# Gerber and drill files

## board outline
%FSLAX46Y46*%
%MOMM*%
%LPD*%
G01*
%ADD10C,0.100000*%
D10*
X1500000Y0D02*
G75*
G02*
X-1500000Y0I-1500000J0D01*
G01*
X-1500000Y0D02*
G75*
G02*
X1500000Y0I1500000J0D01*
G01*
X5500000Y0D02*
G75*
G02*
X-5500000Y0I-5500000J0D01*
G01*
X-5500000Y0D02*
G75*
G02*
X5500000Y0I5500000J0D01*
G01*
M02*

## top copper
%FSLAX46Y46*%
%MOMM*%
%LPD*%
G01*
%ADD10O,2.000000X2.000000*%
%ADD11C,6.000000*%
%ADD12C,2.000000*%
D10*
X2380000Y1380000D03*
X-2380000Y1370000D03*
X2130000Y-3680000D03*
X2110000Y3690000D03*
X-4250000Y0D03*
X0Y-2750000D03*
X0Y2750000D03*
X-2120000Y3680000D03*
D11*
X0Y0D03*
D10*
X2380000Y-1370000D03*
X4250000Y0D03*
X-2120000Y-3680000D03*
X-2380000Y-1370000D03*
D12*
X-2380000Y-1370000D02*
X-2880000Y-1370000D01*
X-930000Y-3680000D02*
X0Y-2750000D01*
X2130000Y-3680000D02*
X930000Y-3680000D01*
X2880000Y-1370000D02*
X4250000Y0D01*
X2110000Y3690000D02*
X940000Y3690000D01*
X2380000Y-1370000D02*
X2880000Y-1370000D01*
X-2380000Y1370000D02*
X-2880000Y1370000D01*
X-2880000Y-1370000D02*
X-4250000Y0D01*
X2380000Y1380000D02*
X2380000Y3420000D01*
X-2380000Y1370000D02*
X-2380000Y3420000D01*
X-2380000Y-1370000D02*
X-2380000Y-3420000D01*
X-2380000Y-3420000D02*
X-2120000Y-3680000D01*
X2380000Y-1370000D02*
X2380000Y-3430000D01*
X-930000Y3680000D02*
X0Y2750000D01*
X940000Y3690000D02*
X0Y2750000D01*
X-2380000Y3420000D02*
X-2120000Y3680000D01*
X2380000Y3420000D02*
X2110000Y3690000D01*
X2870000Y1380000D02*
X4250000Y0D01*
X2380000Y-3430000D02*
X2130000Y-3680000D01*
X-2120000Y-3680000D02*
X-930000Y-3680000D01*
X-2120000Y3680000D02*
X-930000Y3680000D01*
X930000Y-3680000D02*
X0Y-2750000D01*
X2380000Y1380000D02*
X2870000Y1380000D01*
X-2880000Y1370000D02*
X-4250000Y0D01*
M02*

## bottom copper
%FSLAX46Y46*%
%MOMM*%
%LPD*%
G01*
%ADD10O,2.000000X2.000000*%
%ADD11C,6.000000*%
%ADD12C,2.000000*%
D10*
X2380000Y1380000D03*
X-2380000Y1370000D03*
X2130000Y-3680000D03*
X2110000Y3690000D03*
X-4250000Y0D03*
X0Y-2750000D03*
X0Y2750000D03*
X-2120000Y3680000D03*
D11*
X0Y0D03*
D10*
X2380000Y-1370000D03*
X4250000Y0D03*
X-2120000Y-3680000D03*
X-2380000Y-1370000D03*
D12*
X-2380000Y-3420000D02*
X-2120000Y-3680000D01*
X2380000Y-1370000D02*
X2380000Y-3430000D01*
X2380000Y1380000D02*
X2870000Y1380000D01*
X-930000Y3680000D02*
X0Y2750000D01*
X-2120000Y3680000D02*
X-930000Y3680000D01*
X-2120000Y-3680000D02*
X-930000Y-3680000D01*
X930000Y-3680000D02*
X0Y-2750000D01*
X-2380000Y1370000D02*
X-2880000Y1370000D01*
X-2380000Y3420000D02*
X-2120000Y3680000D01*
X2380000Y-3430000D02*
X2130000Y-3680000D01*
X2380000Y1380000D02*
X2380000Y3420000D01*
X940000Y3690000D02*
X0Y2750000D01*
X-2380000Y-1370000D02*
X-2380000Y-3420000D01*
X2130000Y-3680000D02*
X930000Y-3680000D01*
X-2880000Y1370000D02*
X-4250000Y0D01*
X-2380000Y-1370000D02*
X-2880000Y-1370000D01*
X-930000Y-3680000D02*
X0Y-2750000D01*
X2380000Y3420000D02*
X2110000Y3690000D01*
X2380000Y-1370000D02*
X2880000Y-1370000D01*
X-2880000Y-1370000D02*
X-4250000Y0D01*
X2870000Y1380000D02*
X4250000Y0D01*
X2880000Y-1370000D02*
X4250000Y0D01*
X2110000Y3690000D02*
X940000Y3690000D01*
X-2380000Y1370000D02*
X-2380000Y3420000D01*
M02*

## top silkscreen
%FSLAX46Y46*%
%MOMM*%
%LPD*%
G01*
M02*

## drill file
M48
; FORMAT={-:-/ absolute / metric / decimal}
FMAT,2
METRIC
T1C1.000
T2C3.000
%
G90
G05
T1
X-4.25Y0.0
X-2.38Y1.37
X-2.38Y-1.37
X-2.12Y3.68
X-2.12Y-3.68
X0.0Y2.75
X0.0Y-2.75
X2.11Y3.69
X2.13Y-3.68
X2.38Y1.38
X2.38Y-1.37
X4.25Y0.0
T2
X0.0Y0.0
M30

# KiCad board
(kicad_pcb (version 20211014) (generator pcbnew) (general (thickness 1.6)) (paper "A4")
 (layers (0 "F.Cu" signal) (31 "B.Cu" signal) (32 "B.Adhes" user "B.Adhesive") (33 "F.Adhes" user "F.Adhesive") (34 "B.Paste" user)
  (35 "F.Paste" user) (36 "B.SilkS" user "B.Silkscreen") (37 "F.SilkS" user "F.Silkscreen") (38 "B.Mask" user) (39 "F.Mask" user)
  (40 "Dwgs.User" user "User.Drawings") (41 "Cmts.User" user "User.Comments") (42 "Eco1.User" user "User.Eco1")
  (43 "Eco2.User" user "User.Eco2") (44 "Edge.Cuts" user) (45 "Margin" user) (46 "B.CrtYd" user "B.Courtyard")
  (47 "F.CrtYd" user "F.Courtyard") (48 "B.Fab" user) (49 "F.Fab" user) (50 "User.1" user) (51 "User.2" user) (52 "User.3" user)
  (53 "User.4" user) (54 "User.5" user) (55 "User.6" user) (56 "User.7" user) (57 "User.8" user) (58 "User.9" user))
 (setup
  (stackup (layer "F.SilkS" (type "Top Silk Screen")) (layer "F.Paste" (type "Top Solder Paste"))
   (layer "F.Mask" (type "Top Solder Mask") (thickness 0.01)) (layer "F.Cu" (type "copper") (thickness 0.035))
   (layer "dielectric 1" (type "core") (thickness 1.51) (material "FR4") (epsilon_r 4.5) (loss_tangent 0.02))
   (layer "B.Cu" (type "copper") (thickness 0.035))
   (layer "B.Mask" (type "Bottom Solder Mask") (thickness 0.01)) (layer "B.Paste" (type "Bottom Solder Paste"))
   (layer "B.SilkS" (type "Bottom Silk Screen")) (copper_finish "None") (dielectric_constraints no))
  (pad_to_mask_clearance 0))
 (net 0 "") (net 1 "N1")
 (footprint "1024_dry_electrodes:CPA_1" (layer "F.Cu") (at 2.38 -1.38)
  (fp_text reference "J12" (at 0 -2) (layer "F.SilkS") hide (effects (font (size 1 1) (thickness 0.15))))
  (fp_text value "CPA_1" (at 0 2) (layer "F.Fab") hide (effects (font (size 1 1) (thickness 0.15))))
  (pad "1" thru_hole oval (at 0 0) (size 2 2) (drill 1) (layers *.Cu *.Mask) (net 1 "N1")))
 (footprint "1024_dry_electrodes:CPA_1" (layer "F.Cu") (at -2.38 -1.37)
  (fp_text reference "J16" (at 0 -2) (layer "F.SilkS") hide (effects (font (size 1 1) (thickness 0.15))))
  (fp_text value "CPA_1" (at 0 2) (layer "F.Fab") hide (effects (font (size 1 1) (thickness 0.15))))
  (pad "1" thru_hole oval (at 0 0) (size 2 2) (drill 1) (layers *.Cu *.Mask) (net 1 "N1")))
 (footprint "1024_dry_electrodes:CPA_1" (layer "F.Cu") (at 2.13 3.68)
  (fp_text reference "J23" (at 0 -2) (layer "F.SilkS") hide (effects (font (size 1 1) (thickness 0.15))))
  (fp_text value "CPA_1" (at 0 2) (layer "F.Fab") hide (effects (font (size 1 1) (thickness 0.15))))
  (pad "1" thru_hole oval (at 0 0) (size 2 2) (drill 1) (layers *.Cu *.Mask) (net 1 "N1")))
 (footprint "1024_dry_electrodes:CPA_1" (layer "F.Cu") (at 2.11 -3.69)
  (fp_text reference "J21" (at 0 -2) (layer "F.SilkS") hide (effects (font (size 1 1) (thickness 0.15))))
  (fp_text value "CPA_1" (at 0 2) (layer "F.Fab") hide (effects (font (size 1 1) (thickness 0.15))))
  (pad "1" thru_hole oval (at 0 0) (size 2 2) (drill 1) (layers *.Cu *.Mask) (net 1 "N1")))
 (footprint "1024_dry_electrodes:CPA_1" (layer "F.Cu") (at -4.25 0)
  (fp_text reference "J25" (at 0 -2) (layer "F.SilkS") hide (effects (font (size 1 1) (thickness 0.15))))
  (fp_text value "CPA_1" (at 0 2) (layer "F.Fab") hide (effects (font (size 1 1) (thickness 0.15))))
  (pad "1" thru_hole oval (at 0 0) (size 2 2) (drill 1) (layers *.Cu *.Mask) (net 1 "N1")))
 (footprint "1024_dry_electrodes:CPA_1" (layer "F.Cu") (at 0 2.75)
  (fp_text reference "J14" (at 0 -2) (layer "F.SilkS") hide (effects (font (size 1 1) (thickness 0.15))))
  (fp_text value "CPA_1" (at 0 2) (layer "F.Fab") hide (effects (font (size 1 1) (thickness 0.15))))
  (pad "1" thru_hole oval (at 0 0) (size 2 2) (drill 1) (layers *.Cu *.Mask) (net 1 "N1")))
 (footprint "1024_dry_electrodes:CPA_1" (layer "F.Cu") (at 0 -2.75)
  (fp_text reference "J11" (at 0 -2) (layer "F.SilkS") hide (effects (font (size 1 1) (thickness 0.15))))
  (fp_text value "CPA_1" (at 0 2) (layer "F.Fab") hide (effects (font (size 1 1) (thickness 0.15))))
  (pad "1" thru_hole oval (at 0 0) (size 2 2) (drill 1) (layers *.Cu *.Mask) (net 1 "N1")))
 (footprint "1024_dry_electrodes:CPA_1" (layer "F.Cu") (at -2.12 -3.68)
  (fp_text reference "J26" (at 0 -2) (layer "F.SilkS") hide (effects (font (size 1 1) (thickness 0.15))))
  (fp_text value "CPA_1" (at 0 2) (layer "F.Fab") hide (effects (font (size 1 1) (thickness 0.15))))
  (pad "1" thru_hole oval (at 0 0) (size 2 2) (drill 1) (layers *.Cu *.Mask) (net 1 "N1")))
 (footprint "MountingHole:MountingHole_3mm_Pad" (layer "F.Cu") (at 0 0)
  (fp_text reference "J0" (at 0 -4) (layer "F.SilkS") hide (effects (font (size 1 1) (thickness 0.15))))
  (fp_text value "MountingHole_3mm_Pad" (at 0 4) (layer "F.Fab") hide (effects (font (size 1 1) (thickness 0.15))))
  (pad "1" thru_hole circle (at 0 0) (size 6 6) (drill 3) (layers *.Cu *.Mask) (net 1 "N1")))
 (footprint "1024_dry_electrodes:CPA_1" (layer "F.Cu") (at 2.38 1.37)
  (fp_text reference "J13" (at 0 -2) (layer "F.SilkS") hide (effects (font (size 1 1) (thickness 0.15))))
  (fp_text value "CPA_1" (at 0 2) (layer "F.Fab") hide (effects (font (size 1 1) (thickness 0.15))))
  (pad "1" thru_hole oval (at 0 0) (size 2 2) (drill 1) (layers *.Cu *.Mask) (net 1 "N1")))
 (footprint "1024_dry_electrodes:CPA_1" (layer "F.Cu") (at 4.25 0)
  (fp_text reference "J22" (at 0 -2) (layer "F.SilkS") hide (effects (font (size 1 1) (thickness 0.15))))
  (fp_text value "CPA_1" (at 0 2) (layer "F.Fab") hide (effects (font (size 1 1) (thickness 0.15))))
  (pad "1" thru_hole oval (at 0 0) (size 2 2) (drill 1) (layers *.Cu *.Mask) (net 1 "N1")))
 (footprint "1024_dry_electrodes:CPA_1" (layer "F.Cu") (at -2.12 3.68)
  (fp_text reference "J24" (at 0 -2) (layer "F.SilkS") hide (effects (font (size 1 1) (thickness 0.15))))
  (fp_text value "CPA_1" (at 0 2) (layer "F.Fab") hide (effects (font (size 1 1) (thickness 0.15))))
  (pad "1" thru_hole oval (at 0 0) (size 2 2) (drill 1) (layers *.Cu *.Mask) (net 1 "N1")))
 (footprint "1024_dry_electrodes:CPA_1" (layer "F.Cu") (at -2.38 1.37)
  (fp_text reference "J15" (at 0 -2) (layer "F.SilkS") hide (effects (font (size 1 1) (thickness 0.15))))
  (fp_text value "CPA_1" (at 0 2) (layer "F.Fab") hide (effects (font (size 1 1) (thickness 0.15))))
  (pad "1" thru_hole oval (at 0 0) (size 2 2) (drill 1) (layers *.Cu *.Mask) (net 1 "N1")))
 (gr_circle (center 0 0) (end 0 -1.5) (layer "Edge.Cuts") (width 0.1) (fill none))
 (gr_circle (center 0 0) (end 0 -5.5) (layer "Edge.Cuts") (width 0.1) (fill none))
 (segment (start -2.38 1.37) (end -2.88 1.37) (width 2) (layer "F.Cu") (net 1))
 (segment (start -0.93 3.68) (end 0 2.75) (width 2) (layer "F.Cu") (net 1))
 (segment (start 2.13 3.68) (end 0.93 3.68) (width 2) (layer "F.Cu") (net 1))
 (segment (start 2.88 1.37) (end 4.25 0) (width 2) (layer "F.Cu") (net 1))
 (segment (start 2.11 -3.69) (end 0.94 -3.69) (width 2) (layer "F.Cu") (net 1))
 (segment (start 2.38 1.37) (end 2.88 1.37) (width 2) (layer "F.Cu") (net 1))
 (segment (start -2.38 -1.37) (end -2.88 -1.37) (width 2) (layer "F.Cu") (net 1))
 (segment (start -2.88 1.37) (end -4.25 0) (width 2) (layer "F.Cu") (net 1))
 (segment (start 2.38 -1.38) (end 2.38 -3.42) (width 2) (layer "F.Cu") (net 1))
 (segment (start -2.38 -1.37) (end -2.38 -3.42) (width 2) (layer "F.Cu") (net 1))
 (segment (start -2.38 1.37) (end -2.38 3.42) (width 2) (layer "F.Cu") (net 1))
 (segment (start -2.38 3.42) (end -2.12 3.68) (width 2) (layer "F.Cu") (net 1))
 (segment (start 2.38 1.37) (end 2.38 3.43) (width 2) (layer "F.Cu") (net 1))
 (segment (start -0.93 -3.68) (end 0 -2.75) (width 2) (layer "F.Cu") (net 1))
 (segment (start 0.94 -3.69) (end 0 -2.75) (width 2) (layer "F.Cu") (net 1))
 (segment (start -2.38 -3.42) (end -2.12 -3.68) (width 2) (layer "F.Cu") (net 1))
 (segment (start 2.38 -3.42) (end 2.11 -3.69) (width 2) (layer "F.Cu") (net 1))
 (segment (start 2.87 -1.38) (end 4.25 0) (width 2) (layer "F.Cu") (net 1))
 (segment (start 2.38 3.43) (end 2.13 3.68) (width 2) (layer "F.Cu") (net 1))
 (segment (start -2.12 3.68) (end -0.93 3.68) (width 2) (layer "F.Cu") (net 1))
 (segment (start -2.12 -3.68) (end -0.93 -3.68) (width 2) (layer "F.Cu") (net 1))
 (segment (start 0.93 3.68) (end 0 2.75) (width 2) (layer "F.Cu") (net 1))
 (segment (start 2.38 -1.38) (end 2.87 -1.38) (width 2) (layer "F.Cu") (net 1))
 (segment (start -2.88 -1.37) (end -4.25 0) (width 2) (layer "F.Cu") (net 1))
 (segment (start -2.38 3.42) (end -2.12 3.68) (width 2) (layer "B.Cu") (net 1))
 (segment (start 2.38 1.37) (end 2.38 3.43) (width 2) (layer "B.Cu") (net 1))
 (segment (start 2.38 -1.38) (end 2.87 -1.38) (width 2) (layer "B.Cu") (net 1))
 (segment (start -0.93 -3.68) (end 0 -2.75) (width 2) (layer "B.Cu") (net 1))
 (segment (start -2.12 -3.68) (end -0.93 -3.68) (width 2) (layer "B.Cu") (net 1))
 (segment (start -2.12 3.68) (end -0.93 3.68) (width 2) (layer "B.Cu") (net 1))
 (segment (start 0.93 3.68) (end 0 2.75) (width 2) (layer "B.Cu") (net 1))
 (segment (start -2.38 -1.37) (end -2.88 -1.37) (width 2) (layer "B.Cu") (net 1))
 (segment (start -2.38 -3.42) (end -2.12 -3.68) (width 2) (layer "B.Cu") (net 1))
 (segment (start 2.38 3.43) (end 2.13 3.68) (width 2) (layer "B.Cu") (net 1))
 (segment (start 2.38 -1.38) (end 2.38 -3.42) (width 2) (layer "B.Cu") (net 1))
 (segment (start 0.94 -3.69) (end 0 -2.75) (width 2) (layer "B.Cu") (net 1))
 (segment (start -2.38 1.37) (end -2.38 3.42) (width 2) (layer "B.Cu") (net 1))
 (segment (start 2.13 3.68) (end 0.93 3.68) (width 2) (layer "B.Cu") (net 1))
 (segment (start -2.88 -1.37) (end -4.25 0) (width 2) (layer "B.Cu") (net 1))
 (segment (start -2.38 1.37) (end -2.88 1.37) (width 2) (layer "B.Cu") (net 1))
 (segment (start -0.93 3.68) (end 0 2.75) (width 2) (layer "B.Cu") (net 1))
 (segment (start 2.38 -3.42) (end 2.11 -3.69) (width 2) (layer "B.Cu") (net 1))
 (segment (start 2.38 1.37) (end 2.88 1.37) (width 2) (layer "B.Cu") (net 1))
 (segment (start -2.88 1.37) (end -4.25 0) (width 2) (layer "B.Cu") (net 1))
 (segment (start 2.87 -1.38) (end 4.25 0) (width 2) (layer "B.Cu") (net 1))
 (segment (start 2.88 1.37) (end 4.25 0) (width 2) (layer "B.Cu") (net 1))
 (segment (start 2.11 -3.69) (end 0.94 -3.69) (width 2) (layer "B.Cu") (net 1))
 (segment (start -2.38 -1.37) (end -2.38 -3.42) (width 2) (layer "B.Cu") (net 1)))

